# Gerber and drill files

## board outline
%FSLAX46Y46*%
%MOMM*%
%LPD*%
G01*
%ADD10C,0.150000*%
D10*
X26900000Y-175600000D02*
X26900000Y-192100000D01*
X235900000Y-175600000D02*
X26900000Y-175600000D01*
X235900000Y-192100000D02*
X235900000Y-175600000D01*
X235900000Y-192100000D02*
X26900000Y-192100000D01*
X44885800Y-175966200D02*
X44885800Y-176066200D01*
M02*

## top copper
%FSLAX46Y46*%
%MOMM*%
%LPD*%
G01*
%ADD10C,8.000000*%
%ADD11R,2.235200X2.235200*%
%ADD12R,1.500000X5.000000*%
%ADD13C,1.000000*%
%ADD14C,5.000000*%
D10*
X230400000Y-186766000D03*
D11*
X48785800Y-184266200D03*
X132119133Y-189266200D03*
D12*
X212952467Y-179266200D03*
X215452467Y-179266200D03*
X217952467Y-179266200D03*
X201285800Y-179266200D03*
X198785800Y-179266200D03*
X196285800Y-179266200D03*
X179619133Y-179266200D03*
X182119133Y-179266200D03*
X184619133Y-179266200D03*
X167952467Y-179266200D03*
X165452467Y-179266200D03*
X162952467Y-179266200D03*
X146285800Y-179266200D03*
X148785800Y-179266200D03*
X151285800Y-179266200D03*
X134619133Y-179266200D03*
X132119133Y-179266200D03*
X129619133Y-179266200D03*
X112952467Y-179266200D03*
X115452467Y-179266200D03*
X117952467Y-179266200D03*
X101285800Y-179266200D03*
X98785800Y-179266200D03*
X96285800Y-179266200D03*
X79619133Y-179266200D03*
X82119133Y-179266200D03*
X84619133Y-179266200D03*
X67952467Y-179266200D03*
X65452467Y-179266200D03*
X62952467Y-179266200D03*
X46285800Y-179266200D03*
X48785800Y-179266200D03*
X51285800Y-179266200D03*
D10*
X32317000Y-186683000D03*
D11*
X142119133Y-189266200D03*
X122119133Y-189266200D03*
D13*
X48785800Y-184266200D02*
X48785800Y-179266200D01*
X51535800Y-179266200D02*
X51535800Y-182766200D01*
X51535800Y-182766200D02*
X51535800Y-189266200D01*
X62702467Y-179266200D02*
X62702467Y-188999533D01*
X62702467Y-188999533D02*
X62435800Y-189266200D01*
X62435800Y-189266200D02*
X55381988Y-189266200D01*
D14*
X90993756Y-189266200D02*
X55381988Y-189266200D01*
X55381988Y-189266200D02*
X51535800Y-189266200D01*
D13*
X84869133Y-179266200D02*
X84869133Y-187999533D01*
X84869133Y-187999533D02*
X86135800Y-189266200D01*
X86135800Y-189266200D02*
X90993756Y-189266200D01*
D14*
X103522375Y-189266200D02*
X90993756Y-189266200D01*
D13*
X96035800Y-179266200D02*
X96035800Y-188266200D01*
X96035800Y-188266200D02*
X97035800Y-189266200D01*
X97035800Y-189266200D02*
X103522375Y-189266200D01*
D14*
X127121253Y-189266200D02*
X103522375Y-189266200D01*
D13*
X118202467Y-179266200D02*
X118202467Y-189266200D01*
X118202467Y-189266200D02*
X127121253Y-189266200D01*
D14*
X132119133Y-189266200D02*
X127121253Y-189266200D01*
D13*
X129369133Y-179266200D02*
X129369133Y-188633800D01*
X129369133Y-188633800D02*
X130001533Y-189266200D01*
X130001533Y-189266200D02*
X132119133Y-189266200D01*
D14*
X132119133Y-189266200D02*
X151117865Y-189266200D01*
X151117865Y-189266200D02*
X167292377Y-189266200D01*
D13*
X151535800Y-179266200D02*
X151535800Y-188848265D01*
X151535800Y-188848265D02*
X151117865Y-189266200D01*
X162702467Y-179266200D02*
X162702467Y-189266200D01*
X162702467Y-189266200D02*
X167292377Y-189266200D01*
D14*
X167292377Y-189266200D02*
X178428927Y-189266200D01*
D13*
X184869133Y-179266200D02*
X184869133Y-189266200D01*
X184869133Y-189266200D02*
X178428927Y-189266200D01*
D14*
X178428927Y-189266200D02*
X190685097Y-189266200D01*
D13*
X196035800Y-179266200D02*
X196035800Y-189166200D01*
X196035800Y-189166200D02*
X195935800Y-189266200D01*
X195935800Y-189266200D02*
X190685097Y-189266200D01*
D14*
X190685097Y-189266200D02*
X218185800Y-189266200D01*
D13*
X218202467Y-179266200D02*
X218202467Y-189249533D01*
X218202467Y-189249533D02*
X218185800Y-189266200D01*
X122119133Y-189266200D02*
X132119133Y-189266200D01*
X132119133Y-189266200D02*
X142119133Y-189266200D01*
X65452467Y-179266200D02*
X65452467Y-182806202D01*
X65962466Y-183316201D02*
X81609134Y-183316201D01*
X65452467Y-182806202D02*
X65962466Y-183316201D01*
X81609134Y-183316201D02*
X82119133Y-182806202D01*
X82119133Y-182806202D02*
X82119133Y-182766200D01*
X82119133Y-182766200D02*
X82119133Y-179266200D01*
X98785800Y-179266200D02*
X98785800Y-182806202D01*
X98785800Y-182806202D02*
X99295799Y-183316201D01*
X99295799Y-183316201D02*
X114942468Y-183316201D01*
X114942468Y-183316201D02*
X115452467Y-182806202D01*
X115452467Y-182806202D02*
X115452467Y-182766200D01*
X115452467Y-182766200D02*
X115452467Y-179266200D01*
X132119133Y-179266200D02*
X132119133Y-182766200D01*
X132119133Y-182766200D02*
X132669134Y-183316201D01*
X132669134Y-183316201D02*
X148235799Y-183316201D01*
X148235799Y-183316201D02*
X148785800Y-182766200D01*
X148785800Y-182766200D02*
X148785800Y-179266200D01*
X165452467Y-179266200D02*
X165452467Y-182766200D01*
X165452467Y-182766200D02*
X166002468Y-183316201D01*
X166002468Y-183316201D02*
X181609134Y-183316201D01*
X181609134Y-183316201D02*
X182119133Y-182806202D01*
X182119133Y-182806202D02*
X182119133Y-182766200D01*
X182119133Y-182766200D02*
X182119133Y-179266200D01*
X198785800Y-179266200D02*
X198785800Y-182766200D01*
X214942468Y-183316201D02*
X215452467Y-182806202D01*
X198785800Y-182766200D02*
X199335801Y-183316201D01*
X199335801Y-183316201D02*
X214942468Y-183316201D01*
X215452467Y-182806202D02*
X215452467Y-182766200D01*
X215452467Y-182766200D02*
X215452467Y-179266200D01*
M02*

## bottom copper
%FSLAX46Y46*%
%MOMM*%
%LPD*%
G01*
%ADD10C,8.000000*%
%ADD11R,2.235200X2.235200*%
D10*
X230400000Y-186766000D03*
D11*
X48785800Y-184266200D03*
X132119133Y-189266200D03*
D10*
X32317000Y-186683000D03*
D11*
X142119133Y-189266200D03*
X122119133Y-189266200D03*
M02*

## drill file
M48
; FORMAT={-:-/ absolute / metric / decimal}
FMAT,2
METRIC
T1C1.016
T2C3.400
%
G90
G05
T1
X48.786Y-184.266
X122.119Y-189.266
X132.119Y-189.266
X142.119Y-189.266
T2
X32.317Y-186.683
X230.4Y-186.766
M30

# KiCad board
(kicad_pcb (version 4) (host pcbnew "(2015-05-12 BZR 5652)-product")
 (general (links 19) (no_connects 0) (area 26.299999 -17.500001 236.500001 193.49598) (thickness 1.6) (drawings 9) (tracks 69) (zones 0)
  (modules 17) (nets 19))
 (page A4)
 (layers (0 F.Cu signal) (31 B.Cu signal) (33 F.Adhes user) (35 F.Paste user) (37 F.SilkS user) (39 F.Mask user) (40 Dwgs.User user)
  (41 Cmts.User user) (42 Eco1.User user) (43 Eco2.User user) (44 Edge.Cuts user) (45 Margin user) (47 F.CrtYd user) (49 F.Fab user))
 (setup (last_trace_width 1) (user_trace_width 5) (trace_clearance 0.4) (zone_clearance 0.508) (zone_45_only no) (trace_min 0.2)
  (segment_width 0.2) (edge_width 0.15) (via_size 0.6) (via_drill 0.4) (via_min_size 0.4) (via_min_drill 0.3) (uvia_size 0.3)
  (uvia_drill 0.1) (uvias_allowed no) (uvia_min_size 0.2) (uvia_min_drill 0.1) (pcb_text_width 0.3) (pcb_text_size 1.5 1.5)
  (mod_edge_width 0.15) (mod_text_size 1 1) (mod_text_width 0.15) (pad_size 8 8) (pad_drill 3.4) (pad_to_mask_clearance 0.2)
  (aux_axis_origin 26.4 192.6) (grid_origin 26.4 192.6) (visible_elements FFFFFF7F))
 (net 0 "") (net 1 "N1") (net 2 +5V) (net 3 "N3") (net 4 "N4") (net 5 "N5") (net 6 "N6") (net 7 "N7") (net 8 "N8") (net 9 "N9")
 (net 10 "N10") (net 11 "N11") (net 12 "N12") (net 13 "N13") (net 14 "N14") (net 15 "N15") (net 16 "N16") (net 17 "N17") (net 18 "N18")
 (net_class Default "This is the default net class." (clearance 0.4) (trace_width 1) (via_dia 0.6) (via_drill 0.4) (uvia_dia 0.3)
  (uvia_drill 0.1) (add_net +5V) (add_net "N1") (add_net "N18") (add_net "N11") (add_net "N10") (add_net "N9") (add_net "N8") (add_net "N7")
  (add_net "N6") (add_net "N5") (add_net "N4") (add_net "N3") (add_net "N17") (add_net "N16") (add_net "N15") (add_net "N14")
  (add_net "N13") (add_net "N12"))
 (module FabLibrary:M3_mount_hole (layer F.Cu) (at 230.4 186.766)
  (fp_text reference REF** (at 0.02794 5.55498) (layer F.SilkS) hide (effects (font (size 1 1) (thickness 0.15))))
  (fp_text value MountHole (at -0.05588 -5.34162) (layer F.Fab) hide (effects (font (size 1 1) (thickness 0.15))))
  (pad 1 thru_hole circle (at 0 0) (size 8 8) (drill 3.4) (layers *.Cu *.Mask F.SilkS)))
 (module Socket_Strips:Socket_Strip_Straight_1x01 (layer F.Cu) (at 48.7858 184.2662 90)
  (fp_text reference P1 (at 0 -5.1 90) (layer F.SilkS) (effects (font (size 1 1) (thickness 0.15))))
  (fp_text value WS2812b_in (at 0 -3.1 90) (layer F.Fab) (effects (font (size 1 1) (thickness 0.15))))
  (pad 1 thru_hole rect (at 0 0 90) (size 2.2352 2.2352) (drill 1.016) (layers *.Cu *.Mask F.SilkS) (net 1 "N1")))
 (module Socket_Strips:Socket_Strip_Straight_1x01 (layer F.Cu) (at 132.119133 189.2662 90)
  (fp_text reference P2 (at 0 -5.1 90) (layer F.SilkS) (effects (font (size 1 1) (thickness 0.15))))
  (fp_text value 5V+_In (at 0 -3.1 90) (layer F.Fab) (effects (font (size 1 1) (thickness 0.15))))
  (pad 1 thru_hole rect (at 0 0 90) (size 2.2352 2.2352) (drill 1.016) (layers *.Cu *.Mask F.SilkS) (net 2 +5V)))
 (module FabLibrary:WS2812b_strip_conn (layer F.Cu) (at 215.452467 179.2662 270)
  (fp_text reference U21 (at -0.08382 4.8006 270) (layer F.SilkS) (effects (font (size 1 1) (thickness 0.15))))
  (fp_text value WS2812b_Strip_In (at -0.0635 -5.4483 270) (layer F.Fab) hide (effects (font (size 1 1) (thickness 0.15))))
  (pad 1 smd rect (at 0 2.5 270) (size 5 1.5) (layers F.Cu F.Paste F.Mask) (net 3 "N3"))
  (pad 2 smd rect (at 0 0 270) (size 5 1.5) (layers F.Cu F.Paste F.Mask) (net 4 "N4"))
  (pad 3 smd rect (at 0 -2.5 270) (size 5 1.5) (layers F.Cu F.Paste F.Mask) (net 2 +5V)))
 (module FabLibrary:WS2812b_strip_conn (layer F.Cu) (at 198.7858 179.2662 90)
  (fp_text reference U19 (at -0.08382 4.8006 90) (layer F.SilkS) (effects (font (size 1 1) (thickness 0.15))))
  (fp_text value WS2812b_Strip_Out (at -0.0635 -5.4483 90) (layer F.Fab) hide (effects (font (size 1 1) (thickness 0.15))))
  (pad 1 smd rect (at 0 2.5 90) (size 5 1.5) (layers F.Cu F.Paste F.Mask) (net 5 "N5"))
  (pad 2 smd rect (at 0 0 90) (size 5 1.5) (layers F.Cu F.Paste F.Mask) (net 4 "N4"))
  (pad 3 smd rect (at 0 -2.5 90) (size 5 1.5) (layers F.Cu F.Paste F.Mask) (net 2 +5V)))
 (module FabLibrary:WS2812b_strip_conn (layer F.Cu) (at 182.119133 179.2662 270)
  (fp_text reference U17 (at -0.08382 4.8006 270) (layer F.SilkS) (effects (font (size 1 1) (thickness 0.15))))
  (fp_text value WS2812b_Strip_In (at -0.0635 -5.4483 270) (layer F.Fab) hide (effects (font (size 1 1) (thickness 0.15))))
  (pad 1 smd rect (at 0 2.5 270) (size 5 1.5) (layers F.Cu F.Paste F.Mask) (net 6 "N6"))
  (pad 2 smd rect (at 0 0 270) (size 5 1.5) (layers F.Cu F.Paste F.Mask) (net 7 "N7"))
  (pad 3 smd rect (at 0 -2.5 270) (size 5 1.5) (layers F.Cu F.Paste F.Mask) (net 2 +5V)))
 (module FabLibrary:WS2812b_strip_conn (layer F.Cu) (at 165.452467 179.2662 90)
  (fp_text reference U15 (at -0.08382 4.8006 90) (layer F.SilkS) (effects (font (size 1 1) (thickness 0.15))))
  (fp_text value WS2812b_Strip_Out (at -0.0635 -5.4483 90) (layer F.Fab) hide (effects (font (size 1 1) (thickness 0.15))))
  (pad 1 smd rect (at 0 2.5 90) (size 5 1.5) (layers F.Cu F.Paste F.Mask) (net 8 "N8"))
  (pad 2 smd rect (at 0 0 90) (size 5 1.5) (layers F.Cu F.Paste F.Mask) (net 7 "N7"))
  (pad 3 smd rect (at 0 -2.5 90) (size 5 1.5) (layers F.Cu F.Paste F.Mask) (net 2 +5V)))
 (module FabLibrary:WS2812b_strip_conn (layer F.Cu) (at 148.7858 179.2662 270)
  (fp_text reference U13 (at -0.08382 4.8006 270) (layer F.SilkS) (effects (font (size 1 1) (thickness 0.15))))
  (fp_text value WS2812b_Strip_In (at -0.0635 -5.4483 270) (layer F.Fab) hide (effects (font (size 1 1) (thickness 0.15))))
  (pad 1 smd rect (at 0 2.5 270) (size 5 1.5) (layers F.Cu F.Paste F.Mask) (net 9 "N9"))
  (pad 2 smd rect (at 0 0 270) (size 5 1.5) (layers F.Cu F.Paste F.Mask) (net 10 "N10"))
  (pad 3 smd rect (at 0 -2.5 270) (size 5 1.5) (layers F.Cu F.Paste F.Mask) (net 2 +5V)))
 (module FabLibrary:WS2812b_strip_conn (layer F.Cu) (at 132.119133 179.2662 90)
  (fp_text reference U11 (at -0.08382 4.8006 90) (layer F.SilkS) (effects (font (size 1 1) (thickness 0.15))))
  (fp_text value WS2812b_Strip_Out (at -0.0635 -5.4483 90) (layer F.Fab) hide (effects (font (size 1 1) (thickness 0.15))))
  (pad 1 smd rect (at 0 2.5 90) (size 5 1.5) (layers F.Cu F.Paste F.Mask) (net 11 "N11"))
  (pad 2 smd rect (at 0 0 90) (size 5 1.5) (layers F.Cu F.Paste F.Mask) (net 10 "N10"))
  (pad 3 smd rect (at 0 -2.5 90) (size 5 1.5) (layers F.Cu F.Paste F.Mask) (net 2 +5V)))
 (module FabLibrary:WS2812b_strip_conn (layer F.Cu) (at 115.452467 179.2662 270)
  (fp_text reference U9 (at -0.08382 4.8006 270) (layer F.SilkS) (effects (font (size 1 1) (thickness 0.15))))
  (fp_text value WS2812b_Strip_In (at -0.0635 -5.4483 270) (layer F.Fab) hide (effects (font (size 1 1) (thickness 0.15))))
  (pad 1 smd rect (at 0 2.5 270) (size 5 1.5) (layers F.Cu F.Paste F.Mask) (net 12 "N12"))
  (pad 2 smd rect (at 0 0 270) (size 5 1.5) (layers F.Cu F.Paste F.Mask) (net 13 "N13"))
  (pad 3 smd rect (at 0 -2.5 270) (size 5 1.5) (layers F.Cu F.Paste F.Mask) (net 2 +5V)))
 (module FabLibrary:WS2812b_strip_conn (layer F.Cu) (at 98.7858 179.2662 90)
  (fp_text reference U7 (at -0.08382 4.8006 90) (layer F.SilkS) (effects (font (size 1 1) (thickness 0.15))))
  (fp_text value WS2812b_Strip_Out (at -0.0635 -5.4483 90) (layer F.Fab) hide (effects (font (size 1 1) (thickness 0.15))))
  (pad 1 smd rect (at 0 2.5 90) (size 5 1.5) (layers F.Cu F.Paste F.Mask) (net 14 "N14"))
  (pad 2 smd rect (at 0 0 90) (size 5 1.5) (layers F.Cu F.Paste F.Mask) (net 13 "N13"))
  (pad 3 smd rect (at 0 -2.5 90) (size 5 1.5) (layers F.Cu F.Paste F.Mask) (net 2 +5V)))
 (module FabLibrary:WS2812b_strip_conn (layer F.Cu) (at 82.119133 179.2662 270)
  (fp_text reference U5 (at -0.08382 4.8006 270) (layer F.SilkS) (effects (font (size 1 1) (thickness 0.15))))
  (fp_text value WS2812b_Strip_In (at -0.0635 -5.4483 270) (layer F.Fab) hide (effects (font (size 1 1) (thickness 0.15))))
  (pad 1 smd rect (at 0 2.5 270) (size 5 1.5) (layers F.Cu F.Paste F.Mask) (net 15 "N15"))
  (pad 2 smd rect (at 0 0 270) (size 5 1.5) (layers F.Cu F.Paste F.Mask) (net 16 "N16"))
  (pad 3 smd rect (at 0 -2.5 270) (size 5 1.5) (layers F.Cu F.Paste F.Mask) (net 2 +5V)))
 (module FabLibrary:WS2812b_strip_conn (layer F.Cu) (at 65.452467 179.2662 90)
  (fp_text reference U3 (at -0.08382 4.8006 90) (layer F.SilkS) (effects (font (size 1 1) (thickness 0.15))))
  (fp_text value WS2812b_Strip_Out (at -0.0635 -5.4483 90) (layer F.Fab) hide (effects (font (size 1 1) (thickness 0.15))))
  (pad 1 smd rect (at 0 2.5 90) (size 5 1.5) (layers F.Cu F.Paste F.Mask) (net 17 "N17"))
  (pad 2 smd rect (at 0 0 90) (size 5 1.5) (layers F.Cu F.Paste F.Mask) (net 16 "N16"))
  (pad 3 smd rect (at 0 -2.5 90) (size 5 1.5) (layers F.Cu F.Paste F.Mask) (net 2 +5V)))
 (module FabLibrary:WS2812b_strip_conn (layer F.Cu) (at 48.7858 179.2662 270)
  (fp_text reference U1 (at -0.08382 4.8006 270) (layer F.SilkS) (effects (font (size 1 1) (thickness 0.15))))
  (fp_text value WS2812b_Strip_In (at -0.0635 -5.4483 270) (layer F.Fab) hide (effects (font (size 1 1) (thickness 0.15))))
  (pad 1 smd rect (at 0 2.5 270) (size 5 1.5) (layers F.Cu F.Paste F.Mask) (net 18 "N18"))
  (pad 2 smd rect (at 0 0 270) (size 5 1.5) (layers F.Cu F.Paste F.Mask) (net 1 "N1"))
  (pad 3 smd rect (at 0 -2.5 270) (size 5 1.5) (layers F.Cu F.Paste F.Mask) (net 2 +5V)))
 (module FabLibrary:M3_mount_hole (layer F.Cu) (at 32.317 186.683)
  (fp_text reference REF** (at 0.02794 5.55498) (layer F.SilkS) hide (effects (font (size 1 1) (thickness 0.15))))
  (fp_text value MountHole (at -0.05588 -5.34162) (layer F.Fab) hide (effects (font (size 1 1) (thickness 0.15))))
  (pad 1 thru_hole circle (at 0 0) (size 8 8) (drill 3.4) (layers *.Cu *.Mask F.SilkS)))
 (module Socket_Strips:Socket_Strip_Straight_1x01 (layer F.Cu) (at 142.119133 189.2662)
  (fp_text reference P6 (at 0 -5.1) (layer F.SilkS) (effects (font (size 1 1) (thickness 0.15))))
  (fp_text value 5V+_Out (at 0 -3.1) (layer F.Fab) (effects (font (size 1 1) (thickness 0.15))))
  (pad 1 thru_hole rect (at 0 0) (size 2.2352 2.2352) (drill 1.016) (layers *.Cu *.Mask F.SilkS) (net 2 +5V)))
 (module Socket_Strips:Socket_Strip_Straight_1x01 (layer F.Cu) (at 122.119133 189.2662)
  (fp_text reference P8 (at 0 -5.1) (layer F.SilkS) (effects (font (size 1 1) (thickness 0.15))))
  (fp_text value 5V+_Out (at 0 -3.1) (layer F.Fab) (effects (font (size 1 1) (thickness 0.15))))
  (pad 1 thru_hole rect (at 0 0) (size 2.2352 2.2352) (drill 1.016) (layers *.Cu *.Mask F.SilkS) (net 2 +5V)))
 (gr_line (start 26.9 175.6) (end 26.9 192.1) (layer Edge.Cuts) (width 0.15))
 (gr_line (start 235.9 175.6) (end 26.9 175.6) (layer Edge.Cuts) (width 0.15))
 (gr_line (start 235.9 192.1) (end 235.9 175.6) (layer Edge.Cuts) (width 0.15))
 (gr_line (start 235.9 192.1) (end 26.9 192.1) (angle 90) (layer Edge.Cuts) (width 0.15))
 (gr_line (start 44.8858 175.9662) (end 44.8858 176.0662) (angle 90) (layer Edge.Cuts) (width 0.15))
 (segment (start 48.7858 184.2662) (end 48.7858 179.2662) (width 1) (layer F.Cu) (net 1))
 (segment (start 51.5358 179.2662) (end 51.5358 182.7662) (width 1) (layer F.Cu) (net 2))
 (segment (start 51.5358 182.7662) (end 51.5358 189.2662) (width 1) (layer F.Cu) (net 2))
 (segment (start 62.702467 179.2662) (end 62.702467 188.999533) (width 1) (layer F.Cu) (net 2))
 (segment (start 62.702467 188.999533) (end 62.4358 189.2662) (width 1) (layer F.Cu) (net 2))
 (segment (start 62.4358 189.2662) (end 55.381988 189.2662) (width 1) (layer F.Cu) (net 2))
 (segment (start 90.993756 189.2662) (end 55.381988 189.2662) (width 5) (layer F.Cu) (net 2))
 (segment (start 55.381988 189.2662) (end 51.5358 189.2662) (width 5) (layer F.Cu) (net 2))
 (segment (start 84.869133 179.2662) (end 84.869133 187.999533) (width 1) (layer F.Cu) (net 2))
 (segment (start 84.869133 187.999533) (end 86.1358 189.2662) (width 1) (layer F.Cu) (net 2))
 (segment (start 86.1358 189.2662) (end 90.993756 189.2662) (width 1) (layer F.Cu) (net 2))
 (segment (start 103.522375 189.2662) (end 90.993756 189.2662) (width 5) (layer F.Cu) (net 2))
 (segment (start 96.0358 179.2662) (end 96.0358 188.2662) (width 1) (layer F.Cu) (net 2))
 (segment (start 96.0358 188.2662) (end 97.0358 189.2662) (width 1) (layer F.Cu) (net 2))
 (segment (start 97.0358 189.2662) (end 103.522375 189.2662) (width 1) (layer F.Cu) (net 2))
 (segment (start 127.121253 189.2662) (end 103.522375 189.2662) (width 5) (layer F.Cu) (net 2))
 (segment (start 118.202467 179.2662) (end 118.202467 189.2662) (width 1) (layer F.Cu) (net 2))
 (segment (start 118.202467 189.2662) (end 127.121253 189.2662) (width 1) (layer F.Cu) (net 2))
 (segment (start 132.119133 189.2662) (end 127.121253 189.2662) (width 5) (layer F.Cu) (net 2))
 (segment (start 129.369133 179.2662) (end 129.369133 188.6338) (width 1) (layer F.Cu) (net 2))
 (segment (start 129.369133 188.6338) (end 130.001533 189.2662) (width 1) (layer F.Cu) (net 2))
 (segment (start 130.001533 189.2662) (end 132.119133 189.2662) (width 1) (layer F.Cu) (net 2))
 (segment (start 132.119133 189.2662) (end 151.117865 189.2662) (width 5) (layer F.Cu) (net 2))
 (segment (start 151.117865 189.2662) (end 167.292377 189.2662) (width 5) (layer F.Cu) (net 2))
 (segment (start 151.5358 179.2662) (end 151.5358 188.848265) (width 1) (layer F.Cu) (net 2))
 (segment (start 151.5358 188.848265) (end 151.117865 189.2662) (width 1) (layer F.Cu) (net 2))
 (segment (start 162.702467 179.2662) (end 162.702467 189.2662) (width 1) (layer F.Cu) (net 2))
 (segment (start 162.702467 189.2662) (end 167.292377 189.2662) (width 1) (layer F.Cu) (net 2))
 (segment (start 167.292377 189.2662) (end 178.428927 189.2662) (width 5) (layer F.Cu) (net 2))
 (segment (start 184.869133 179.2662) (end 184.869133 189.2662) (width 1) (layer F.Cu) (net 2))
 (segment (start 184.869133 189.2662) (end 178.428927 189.2662) (width 1) (layer F.Cu) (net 2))
 (segment (start 178.428927 189.2662) (end 190.685097 189.2662) (width 5) (layer F.Cu) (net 2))
 (segment (start 196.0358 179.2662) (end 196.0358 189.1662) (width 1) (layer F.Cu) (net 2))
 (segment (start 196.0358 189.1662) (end 195.9358 189.2662) (width 1) (layer F.Cu) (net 2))
 (segment (start 195.9358 189.2662) (end 190.685097 189.2662) (width 1) (layer F.Cu) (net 2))
 (segment (start 190.685097 189.2662) (end 218.1858 189.2662) (width 5) (layer F.Cu) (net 2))
 (segment (start 218.202467 179.2662) (end 218.202467 189.249533) (width 1) (layer F.Cu) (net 2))
 (segment (start 218.202467 189.249533) (end 218.1858 189.2662) (width 1) (layer F.Cu) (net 2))
 (segment (start 122.119133 189.2662) (end 132.119133 189.2662) (width 1) (layer F.Cu) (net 2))
 (segment (start 132.119133 189.2662) (end 142.119133 189.2662) (width 1) (layer F.Cu) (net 2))
 (segment (start 65.452467 179.2662) (end 65.452467 182.806202) (width 1) (layer F.Cu) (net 16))
 (segment (start 65.962466 183.316201) (end 81.609134 183.316201) (width 1) (layer F.Cu) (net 16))
 (segment (start 65.452467 182.806202) (end 65.962466 183.316201) (width 1) (layer F.Cu) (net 16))
 (segment (start 81.609134 183.316201) (end 82.119133 182.806202) (width 1) (layer F.Cu) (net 16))
 (segment (start 82.119133 182.806202) (end 82.119133 182.7662) (width 1) (layer F.Cu) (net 16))
 (segment (start 82.119133 182.7662) (end 82.119133 179.2662) (width 1) (layer F.Cu) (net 16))
 (segment (start 98.7858 179.2662) (end 98.7858 182.806202) (width 1) (layer F.Cu) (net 13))
 (segment (start 98.7858 182.806202) (end 99.295799 183.316201) (width 1) (layer F.Cu) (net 13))
 (segment (start 99.295799 183.316201) (end 114.942468 183.316201) (width 1) (layer F.Cu) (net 13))
 (segment (start 114.942468 183.316201) (end 115.452467 182.806202) (width 1) (layer F.Cu) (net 13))
 (segment (start 115.452467 182.806202) (end 115.452467 182.7662) (width 1) (layer F.Cu) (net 13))
 (segment (start 115.452467 182.7662) (end 115.452467 179.2662) (width 1) (layer F.Cu) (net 13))
 (segment (start 132.119133 179.2662) (end 132.119133 182.7662) (width 1) (layer F.Cu) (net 10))
 (segment (start 132.119133 182.7662) (end 132.669134 183.316201) (width 1) (layer F.Cu) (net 10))
 (segment (start 132.669134 183.316201) (end 148.235799 183.316201) (width 1) (layer F.Cu) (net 10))
 (segment (start 148.235799 183.316201) (end 148.7858 182.7662) (width 1) (layer F.Cu) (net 10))
 (segment (start 148.7858 182.7662) (end 148.7858 179.2662) (width 1) (layer F.Cu) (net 10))
 (segment (start 165.452467 179.2662) (end 165.452467 182.7662) (width 1) (layer F.Cu) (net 7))
 (segment (start 165.452467 182.7662) (end 166.002468 183.316201) (width 1) (layer F.Cu) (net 7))
 (segment (start 166.002468 183.316201) (end 181.609134 183.316201) (width 1) (layer F.Cu) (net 7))
 (segment (start 181.609134 183.316201) (end 182.119133 182.806202) (width 1) (layer F.Cu) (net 7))
 (segment (start 182.119133 182.806202) (end 182.119133 182.7662) (width 1) (layer F.Cu) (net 7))
 (segment (start 182.119133 182.7662) (end 182.119133 179.2662) (width 1) (layer F.Cu) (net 7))
 (segment (start 198.7858 179.2662) (end 198.7858 182.7662) (width 1) (layer F.Cu) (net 4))
 (segment (start 214.942468 183.316201) (end 215.452467 182.806202) (width 1) (layer F.Cu) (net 4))
 (segment (start 198.7858 182.7662) (end 199.335801 183.316201) (width 1) (layer F.Cu) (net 4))
 (segment (start 199.335801 183.316201) (end 214.942468 183.316201) (width 1) (layer F.Cu) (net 4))
 (segment (start 215.452467 182.806202) (end 215.452467 182.7662) (width 1) (layer F.Cu) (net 4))
 (segment (start 215.452467 182.7662) (end 215.452467 179.2662) (width 1) (layer F.Cu) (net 4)))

